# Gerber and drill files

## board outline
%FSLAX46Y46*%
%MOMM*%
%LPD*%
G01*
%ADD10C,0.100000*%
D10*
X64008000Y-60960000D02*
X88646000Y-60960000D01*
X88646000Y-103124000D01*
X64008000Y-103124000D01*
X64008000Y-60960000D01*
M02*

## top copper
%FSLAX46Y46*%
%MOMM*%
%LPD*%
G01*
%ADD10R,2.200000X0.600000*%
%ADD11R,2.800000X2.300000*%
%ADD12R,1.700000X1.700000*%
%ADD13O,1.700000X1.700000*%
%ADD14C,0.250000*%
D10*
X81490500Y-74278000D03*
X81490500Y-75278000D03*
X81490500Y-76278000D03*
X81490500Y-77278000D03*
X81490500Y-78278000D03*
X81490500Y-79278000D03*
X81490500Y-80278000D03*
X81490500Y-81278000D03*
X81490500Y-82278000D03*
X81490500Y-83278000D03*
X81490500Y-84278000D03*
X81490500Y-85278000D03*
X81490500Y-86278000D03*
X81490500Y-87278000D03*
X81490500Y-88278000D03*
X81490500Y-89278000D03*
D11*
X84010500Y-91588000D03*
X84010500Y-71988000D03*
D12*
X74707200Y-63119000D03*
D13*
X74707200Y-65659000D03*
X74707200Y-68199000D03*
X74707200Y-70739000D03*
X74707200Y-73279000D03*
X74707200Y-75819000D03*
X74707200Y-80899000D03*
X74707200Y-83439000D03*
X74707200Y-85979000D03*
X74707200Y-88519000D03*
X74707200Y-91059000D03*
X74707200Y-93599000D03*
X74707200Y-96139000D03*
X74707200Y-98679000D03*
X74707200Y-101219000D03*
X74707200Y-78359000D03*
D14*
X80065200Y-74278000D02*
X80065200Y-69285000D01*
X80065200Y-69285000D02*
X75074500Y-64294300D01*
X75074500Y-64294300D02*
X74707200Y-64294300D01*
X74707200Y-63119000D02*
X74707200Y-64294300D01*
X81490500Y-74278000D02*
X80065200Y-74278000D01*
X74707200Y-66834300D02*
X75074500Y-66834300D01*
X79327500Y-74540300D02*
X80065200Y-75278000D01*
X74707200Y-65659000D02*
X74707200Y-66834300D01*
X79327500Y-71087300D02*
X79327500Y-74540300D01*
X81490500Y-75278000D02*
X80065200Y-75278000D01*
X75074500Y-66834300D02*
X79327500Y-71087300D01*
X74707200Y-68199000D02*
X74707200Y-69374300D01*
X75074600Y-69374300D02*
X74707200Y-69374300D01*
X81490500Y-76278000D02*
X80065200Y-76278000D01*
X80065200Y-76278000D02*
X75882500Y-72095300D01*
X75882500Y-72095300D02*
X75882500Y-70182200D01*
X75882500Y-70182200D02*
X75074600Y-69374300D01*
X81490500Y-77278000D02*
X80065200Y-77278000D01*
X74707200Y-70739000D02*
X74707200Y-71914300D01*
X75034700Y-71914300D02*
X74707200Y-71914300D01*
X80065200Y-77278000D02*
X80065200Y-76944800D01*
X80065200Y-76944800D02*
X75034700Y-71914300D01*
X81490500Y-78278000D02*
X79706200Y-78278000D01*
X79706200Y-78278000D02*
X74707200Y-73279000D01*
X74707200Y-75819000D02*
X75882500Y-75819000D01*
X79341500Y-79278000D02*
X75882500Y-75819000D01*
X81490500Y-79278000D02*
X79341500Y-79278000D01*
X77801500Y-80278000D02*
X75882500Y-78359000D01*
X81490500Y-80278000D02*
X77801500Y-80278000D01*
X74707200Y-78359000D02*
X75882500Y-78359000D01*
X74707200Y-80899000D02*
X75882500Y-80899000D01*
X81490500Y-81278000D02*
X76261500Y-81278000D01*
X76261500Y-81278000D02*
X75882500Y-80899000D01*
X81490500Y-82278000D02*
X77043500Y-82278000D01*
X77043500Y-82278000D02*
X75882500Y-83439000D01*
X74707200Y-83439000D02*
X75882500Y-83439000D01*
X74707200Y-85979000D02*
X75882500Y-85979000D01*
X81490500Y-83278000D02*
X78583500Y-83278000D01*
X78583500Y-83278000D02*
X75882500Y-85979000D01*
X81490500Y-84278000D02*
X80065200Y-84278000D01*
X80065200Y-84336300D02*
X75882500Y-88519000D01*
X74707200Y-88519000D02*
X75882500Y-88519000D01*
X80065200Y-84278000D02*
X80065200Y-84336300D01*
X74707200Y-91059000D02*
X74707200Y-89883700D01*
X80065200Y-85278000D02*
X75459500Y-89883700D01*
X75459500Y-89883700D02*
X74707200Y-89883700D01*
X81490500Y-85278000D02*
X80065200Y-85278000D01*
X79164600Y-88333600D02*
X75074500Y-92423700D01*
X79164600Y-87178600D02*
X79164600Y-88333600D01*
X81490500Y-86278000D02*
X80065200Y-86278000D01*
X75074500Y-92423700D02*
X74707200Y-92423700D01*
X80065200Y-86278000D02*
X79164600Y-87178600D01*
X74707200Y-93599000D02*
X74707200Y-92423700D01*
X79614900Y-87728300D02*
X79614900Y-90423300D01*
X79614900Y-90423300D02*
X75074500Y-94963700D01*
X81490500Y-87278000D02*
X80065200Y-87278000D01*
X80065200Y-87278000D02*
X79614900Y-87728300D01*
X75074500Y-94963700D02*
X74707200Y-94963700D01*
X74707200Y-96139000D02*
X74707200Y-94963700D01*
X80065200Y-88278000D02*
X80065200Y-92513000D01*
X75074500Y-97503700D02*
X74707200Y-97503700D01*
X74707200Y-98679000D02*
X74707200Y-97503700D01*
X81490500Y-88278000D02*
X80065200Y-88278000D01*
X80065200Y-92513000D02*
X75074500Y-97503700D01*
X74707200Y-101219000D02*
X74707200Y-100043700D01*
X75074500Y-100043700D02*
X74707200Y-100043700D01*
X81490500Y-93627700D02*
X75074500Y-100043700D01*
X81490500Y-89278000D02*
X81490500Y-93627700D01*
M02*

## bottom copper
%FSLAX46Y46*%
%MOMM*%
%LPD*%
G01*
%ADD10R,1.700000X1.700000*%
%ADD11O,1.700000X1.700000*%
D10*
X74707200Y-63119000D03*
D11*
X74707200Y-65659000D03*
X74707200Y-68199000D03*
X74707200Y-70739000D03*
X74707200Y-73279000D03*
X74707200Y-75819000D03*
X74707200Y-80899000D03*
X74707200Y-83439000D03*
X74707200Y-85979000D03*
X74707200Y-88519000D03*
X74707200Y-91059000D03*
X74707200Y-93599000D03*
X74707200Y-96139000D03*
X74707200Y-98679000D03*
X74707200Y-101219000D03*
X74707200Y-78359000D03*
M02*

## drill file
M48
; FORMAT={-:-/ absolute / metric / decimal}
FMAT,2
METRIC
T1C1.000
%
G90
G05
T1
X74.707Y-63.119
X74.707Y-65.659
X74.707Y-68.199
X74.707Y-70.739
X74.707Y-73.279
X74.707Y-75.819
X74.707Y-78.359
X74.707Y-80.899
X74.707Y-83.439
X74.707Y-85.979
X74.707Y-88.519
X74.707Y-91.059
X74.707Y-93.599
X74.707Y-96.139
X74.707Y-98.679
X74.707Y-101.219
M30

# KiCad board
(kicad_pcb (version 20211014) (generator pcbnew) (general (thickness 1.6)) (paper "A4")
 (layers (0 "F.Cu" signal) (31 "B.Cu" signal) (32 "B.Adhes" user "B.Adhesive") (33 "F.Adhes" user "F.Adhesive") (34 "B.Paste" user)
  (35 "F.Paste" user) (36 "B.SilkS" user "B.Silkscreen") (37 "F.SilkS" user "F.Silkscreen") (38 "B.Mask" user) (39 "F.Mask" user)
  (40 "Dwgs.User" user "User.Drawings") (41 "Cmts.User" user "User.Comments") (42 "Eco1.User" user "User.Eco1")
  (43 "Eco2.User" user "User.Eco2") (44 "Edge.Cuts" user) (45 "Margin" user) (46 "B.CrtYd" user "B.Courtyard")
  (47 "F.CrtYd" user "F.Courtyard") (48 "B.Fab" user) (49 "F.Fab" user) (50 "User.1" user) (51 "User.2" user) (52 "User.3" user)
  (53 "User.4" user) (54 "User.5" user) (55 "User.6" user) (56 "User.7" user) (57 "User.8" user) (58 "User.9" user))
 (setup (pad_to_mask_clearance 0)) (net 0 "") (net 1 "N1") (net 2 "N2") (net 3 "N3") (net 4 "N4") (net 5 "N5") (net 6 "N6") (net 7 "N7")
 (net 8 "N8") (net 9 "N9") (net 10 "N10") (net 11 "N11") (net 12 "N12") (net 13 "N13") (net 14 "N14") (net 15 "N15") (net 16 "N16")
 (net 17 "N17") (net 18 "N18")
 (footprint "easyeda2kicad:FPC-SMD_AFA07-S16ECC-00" (layer "F.Cu") (at 82.7505 81.788 90)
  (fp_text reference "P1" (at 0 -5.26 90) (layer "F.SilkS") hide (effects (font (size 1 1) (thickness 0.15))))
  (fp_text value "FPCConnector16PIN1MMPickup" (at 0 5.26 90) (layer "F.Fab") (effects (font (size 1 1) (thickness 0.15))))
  (pad "1" smd rect locked (at 7.51 -1.26 270) (size 0.6 2.2) (layers "F.Cu" "F.Paste" "F.Mask") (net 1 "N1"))
  (pad "2" smd rect locked (at 6.51 -1.26 270) (size 0.6 2.2) (layers "F.Cu" "F.Paste" "F.Mask") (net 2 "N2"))
  (pad "3" smd rect locked (at 5.51 -1.26 270) (size 0.6 2.2) (layers "F.Cu" "F.Paste" "F.Mask") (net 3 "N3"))
  (pad "4" smd rect locked (at 4.51 -1.26 270) (size 0.6 2.2) (layers "F.Cu" "F.Paste" "F.Mask") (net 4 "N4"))
  (pad "5" smd rect locked (at 3.51 -1.26 270) (size 0.6 2.2) (layers "F.Cu" "F.Paste" "F.Mask") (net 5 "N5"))
  (pad "6" smd rect locked (at 2.51 -1.26 270) (size 0.6 2.2) (layers "F.Cu" "F.Paste" "F.Mask") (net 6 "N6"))
  (pad "7" smd rect locked (at 1.51 -1.26 270) (size 0.6 2.2) (layers "F.Cu" "F.Paste" "F.Mask") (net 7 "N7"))
  (pad "8" smd rect locked (at 0.51 -1.26 270) (size 0.6 2.2) (layers "F.Cu" "F.Paste" "F.Mask") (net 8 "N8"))
  (pad "9" smd rect locked (at -0.49 -1.26 270) (size 0.6 2.2) (layers "F.Cu" "F.Paste" "F.Mask") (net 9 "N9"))
  (pad "10" smd rect locked (at -1.49 -1.26 270) (size 0.6 2.2) (layers "F.Cu" "F.Paste" "F.Mask") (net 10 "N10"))
  (pad "11" smd rect locked (at -2.49 -1.26 270) (size 0.6 2.2) (layers "F.Cu" "F.Paste" "F.Mask") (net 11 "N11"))
  (pad "12" smd rect locked (at -3.49 -1.26 270) (size 0.6 2.2) (layers "F.Cu" "F.Paste" "F.Mask") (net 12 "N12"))
  (pad "13" smd rect locked (at -4.49 -1.26 270) (size 0.6 2.2) (layers "F.Cu" "F.Paste" "F.Mask") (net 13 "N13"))
  (pad "14" smd rect locked (at -5.49 -1.26 270) (size 0.6 2.2) (layers "F.Cu" "F.Paste" "F.Mask") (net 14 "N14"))
  (pad "15" smd rect locked (at -6.49 -1.26 270) (size 0.6 2.2) (layers "F.Cu" "F.Paste" "F.Mask") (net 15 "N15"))
  (pad "16" smd rect locked (at -7.49 -1.26 270) (size 0.6 2.2) (layers "F.Cu" "F.Paste" "F.Mask") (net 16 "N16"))
  (pad "17" smd rect locked (at -9.8 1.26) (size 2.8 2.3) (layers "F.Cu" "F.Paste" "F.Mask") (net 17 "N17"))
  (pad "18" smd rect locked (at 9.8 1.26) (size 2.8 2.3) (layers "F.Cu" "F.Paste" "F.Mask") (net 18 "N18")))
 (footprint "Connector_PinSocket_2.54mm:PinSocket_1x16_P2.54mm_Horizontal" (layer "F.Cu") (at 74.7072 63.119)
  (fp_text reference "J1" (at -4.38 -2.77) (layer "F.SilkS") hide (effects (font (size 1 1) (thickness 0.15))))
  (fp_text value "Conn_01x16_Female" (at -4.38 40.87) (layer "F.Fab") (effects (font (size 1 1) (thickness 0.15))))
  (pad "1" thru_hole rect (at 0 0) (size 1.7 1.7) (drill 1) (layers *.Cu *.Mask) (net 1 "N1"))
  (pad "2" thru_hole oval (at 0 2.54) (size 1.7 1.7) (drill 1) (layers *.Cu *.Mask) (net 2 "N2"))
  (pad "3" thru_hole oval (at 0 5.08) (size 1.7 1.7) (drill 1) (layers *.Cu *.Mask) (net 3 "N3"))
  (pad "4" thru_hole oval (at 0 7.62) (size 1.7 1.7) (drill 1) (layers *.Cu *.Mask) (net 4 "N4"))
  (pad "5" thru_hole oval (at 0 10.16) (size 1.7 1.7) (drill 1) (layers *.Cu *.Mask) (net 5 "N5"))
  (pad "6" thru_hole oval (at 0 12.7) (size 1.7 1.7) (drill 1) (layers *.Cu *.Mask) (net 6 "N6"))
  (pad "8" thru_hole oval (at 0 17.78) (size 1.7 1.7) (drill 1) (layers *.Cu *.Mask) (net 8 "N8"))
  (pad "9" thru_hole oval (at 0 20.32) (size 1.7 1.7) (drill 1) (layers *.Cu *.Mask) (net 9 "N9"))
  (pad "10" thru_hole oval (at 0 22.86) (size 1.7 1.7) (drill 1) (layers *.Cu *.Mask) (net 10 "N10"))
  (pad "11" thru_hole oval (at 0 25.4) (size 1.7 1.7) (drill 1) (layers *.Cu *.Mask) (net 11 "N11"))
  (pad "12" thru_hole oval (at 0 27.94) (size 1.7 1.7) (drill 1) (layers *.Cu *.Mask) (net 12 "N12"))
  (pad "13" thru_hole oval (at 0 30.48) (size 1.7 1.7) (drill 1) (layers *.Cu *.Mask) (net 13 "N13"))
  (pad "14" thru_hole oval (at 0 33.02) (size 1.7 1.7) (drill 1) (layers *.Cu *.Mask) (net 14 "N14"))
  (pad "15" thru_hole oval (at 0 35.56) (size 1.7 1.7) (drill 1) (layers *.Cu *.Mask) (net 15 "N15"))
  (pad "16" thru_hole oval (at 0 38.1) (size 1.7 1.7) (drill 1) (layers *.Cu *.Mask) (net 16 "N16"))
  (pad "e" thru_hole oval (at 0 15.24) (size 1.7 1.7) (drill 1) (layers *.Cu *.Mask) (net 7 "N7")))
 (gr_rect (start 64.008 103.124) (end 88.646 60.96) (layer "Edge.Cuts") (width 0.1) (fill none))
 (segment (start 80.0652 74.278) (end 80.0652 69.285) (width 0.25) (layer "F.Cu") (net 1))
 (segment (start 80.0652 69.285) (end 75.0745 64.2943) (width 0.25) (layer "F.Cu") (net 1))
 (segment (start 75.0745 64.2943) (end 74.7072 64.2943) (width 0.25) (layer "F.Cu") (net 1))
 (segment (start 74.7072 63.119) (end 74.7072 64.2943) (width 0.25) (layer "F.Cu") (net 1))
 (segment (start 81.4905 74.278) (end 80.0652 74.278) (width 0.25) (layer "F.Cu") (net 1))
 (segment (start 74.7072 66.8343) (end 75.0745 66.8343) (width 0.25) (layer "F.Cu") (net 2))
 (segment (start 79.3275 74.5403) (end 80.0652 75.278) (width 0.25) (layer "F.Cu") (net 2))
 (segment (start 74.7072 65.659) (end 74.7072 66.8343) (width 0.25) (layer "F.Cu") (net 2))
 (segment (start 79.3275 71.0873) (end 79.3275 74.5403) (width 0.25) (layer "F.Cu") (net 2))
 (segment (start 81.4905 75.278) (end 80.0652 75.278) (width 0.25) (layer "F.Cu") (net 2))
 (segment (start 75.0745 66.8343) (end 79.3275 71.0873) (width 0.25) (layer "F.Cu") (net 2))
 (segment (start 74.7072 68.199) (end 74.7072 69.3743) (width 0.25) (layer "F.Cu") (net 3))
 (segment (start 75.0746 69.3743) (end 74.7072 69.3743) (width 0.25) (layer "F.Cu") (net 3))
 (segment (start 81.4905 76.278) (end 80.0652 76.278) (width 0.25) (layer "F.Cu") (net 3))
 (segment (start 80.0652 76.278) (end 75.8825 72.0953) (width 0.25) (layer "F.Cu") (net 3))
 (segment (start 75.8825 72.0953) (end 75.8825 70.1822) (width 0.25) (layer "F.Cu") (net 3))
 (segment (start 75.8825 70.1822) (end 75.0746 69.3743) (width 0.25) (layer "F.Cu") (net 3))
 (segment (start 81.4905 77.278) (end 80.0652 77.278) (width 0.25) (layer "F.Cu") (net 4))
 (segment (start 74.7072 70.739) (end 74.7072 71.9143) (width 0.25) (layer "F.Cu") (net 4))
 (segment (start 75.0347 71.9143) (end 74.7072 71.9143) (width 0.25) (layer "F.Cu") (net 4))
 (segment (start 80.0652 77.278) (end 80.0652 76.9448) (width 0.25) (layer "F.Cu") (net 4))
 (segment (start 80.0652 76.9448) (end 75.0347 71.9143) (width 0.25) (layer "F.Cu") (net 4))
 (segment (start 81.4905 78.278) (end 79.7062 78.278) (width 0.25) (layer "F.Cu") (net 5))
 (segment (start 79.7062 78.278) (end 74.7072 73.279) (width 0.25) (layer "F.Cu") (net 5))
 (segment (start 74.7072 75.819) (end 75.8825 75.819) (width 0.25) (layer "F.Cu") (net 6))
 (segment (start 79.3415 79.278) (end 75.8825 75.819) (width 0.25) (layer "F.Cu") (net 6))
 (segment (start 81.4905 79.278) (end 79.3415 79.278) (width 0.25) (layer "F.Cu") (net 6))
 (segment (start 77.8015 80.278) (end 75.8825 78.359) (width 0.25) (layer "F.Cu") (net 7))
 (segment (start 81.4905 80.278) (end 77.8015 80.278) (width 0.25) (layer "F.Cu") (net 7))
 (segment (start 74.7072 78.359) (end 75.8825 78.359) (width 0.25) (layer "F.Cu") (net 7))
 (segment (start 74.7072 80.899) (end 75.8825 80.899) (width 0.25) (layer "F.Cu") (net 8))
 (segment (start 81.4905 81.278) (end 76.2615 81.278) (width 0.25) (layer "F.Cu") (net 8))
 (segment (start 76.2615 81.278) (end 75.8825 80.899) (width 0.25) (layer "F.Cu") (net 8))
 (segment (start 81.4905 82.278) (end 77.0435 82.278) (width 0.25) (layer "F.Cu") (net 9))
 (segment (start 77.0435 82.278) (end 75.8825 83.439) (width 0.25) (layer "F.Cu") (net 9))
 (segment (start 74.7072 83.439) (end 75.8825 83.439) (width 0.25) (layer "F.Cu") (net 9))
 (segment (start 74.7072 85.979) (end 75.8825 85.979) (width 0.25) (layer "F.Cu") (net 10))
 (segment (start 81.4905 83.278) (end 78.5835 83.278) (width 0.25) (layer "F.Cu") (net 10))
 (segment (start 78.5835 83.278) (end 75.8825 85.979) (width 0.25) (layer "F.Cu") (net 10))
 (segment (start 81.4905 84.278) (end 80.0652 84.278) (width 0.25) (layer "F.Cu") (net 11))
 (segment (start 80.0652 84.3363) (end 75.8825 88.519) (width 0.25) (layer "F.Cu") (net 11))
 (segment (start 74.7072 88.519) (end 75.8825 88.519) (width 0.25) (layer "F.Cu") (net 11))
 (segment (start 80.0652 84.278) (end 80.0652 84.3363) (width 0.25) (layer "F.Cu") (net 11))
 (segment (start 74.7072 91.059) (end 74.7072 89.8837) (width 0.25) (layer "F.Cu") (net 12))
 (segment (start 80.0652 85.278) (end 75.4595 89.8837) (width 0.25) (layer "F.Cu") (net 12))
 (segment (start 75.4595 89.8837) (end 74.7072 89.8837) (width 0.25) (layer "F.Cu") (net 12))
 (segment (start 81.4905 85.278) (end 80.0652 85.278) (width 0.25) (layer "F.Cu") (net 12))
 (segment (start 79.1646 88.3336) (end 75.0745 92.4237) (width 0.25) (layer "F.Cu") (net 13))
 (segment (start 79.1646 87.1786) (end 79.1646 88.3336) (width 0.25) (layer "F.Cu") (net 13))
 (segment (start 81.4905 86.278) (end 80.0652 86.278) (width 0.25) (layer "F.Cu") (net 13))
 (segment (start 75.0745 92.4237) (end 74.7072 92.4237) (width 0.25) (layer "F.Cu") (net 13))
 (segment (start 80.0652 86.278) (end 79.1646 87.1786) (width 0.25) (layer "F.Cu") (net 13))
 (segment (start 74.7072 93.599) (end 74.7072 92.4237) (width 0.25) (layer "F.Cu") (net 13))
 (segment (start 79.6149 87.7283) (end 79.6149 90.4233) (width 0.25) (layer "F.Cu") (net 14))
 (segment (start 79.6149 90.4233) (end 75.0745 94.9637) (width 0.25) (layer "F.Cu") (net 14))
 (segment (start 81.4905 87.278) (end 80.0652 87.278) (width 0.25) (layer "F.Cu") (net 14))
 (segment (start 80.0652 87.278) (end 79.6149 87.7283) (width 0.25) (layer "F.Cu") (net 14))
 (segment (start 75.0745 94.9637) (end 74.7072 94.9637) (width 0.25) (layer "F.Cu") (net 14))
 (segment (start 74.7072 96.139) (end 74.7072 94.9637) (width 0.25) (layer "F.Cu") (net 14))
 (segment (start 80.0652 88.278) (end 80.0652 92.513) (width 0.25) (layer "F.Cu") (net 15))
 (segment (start 75.0745 97.5037) (end 74.7072 97.5037) (width 0.25) (layer "F.Cu") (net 15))
 (segment (start 74.7072 98.679) (end 74.7072 97.5037) (width 0.25) (layer "F.Cu") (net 15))
 (segment (start 81.4905 88.278) (end 80.0652 88.278) (width 0.25) (layer "F.Cu") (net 15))
 (segment (start 80.0652 92.513) (end 75.0745 97.5037) (width 0.25) (layer "F.Cu") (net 15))
 (segment (start 74.7072 101.219) (end 74.7072 100.0437) (width 0.25) (layer "F.Cu") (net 16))
 (segment (start 75.0745 100.0437) (end 74.7072 100.0437) (width 0.25) (layer "F.Cu") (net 16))
 (segment (start 81.4905 93.6277) (end 75.0745 100.0437) (width 0.25) (layer "F.Cu") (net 16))
 (segment (start 81.4905 89.278) (end 81.4905 93.6277) (width 0.25) (layer "F.Cu") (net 16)))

